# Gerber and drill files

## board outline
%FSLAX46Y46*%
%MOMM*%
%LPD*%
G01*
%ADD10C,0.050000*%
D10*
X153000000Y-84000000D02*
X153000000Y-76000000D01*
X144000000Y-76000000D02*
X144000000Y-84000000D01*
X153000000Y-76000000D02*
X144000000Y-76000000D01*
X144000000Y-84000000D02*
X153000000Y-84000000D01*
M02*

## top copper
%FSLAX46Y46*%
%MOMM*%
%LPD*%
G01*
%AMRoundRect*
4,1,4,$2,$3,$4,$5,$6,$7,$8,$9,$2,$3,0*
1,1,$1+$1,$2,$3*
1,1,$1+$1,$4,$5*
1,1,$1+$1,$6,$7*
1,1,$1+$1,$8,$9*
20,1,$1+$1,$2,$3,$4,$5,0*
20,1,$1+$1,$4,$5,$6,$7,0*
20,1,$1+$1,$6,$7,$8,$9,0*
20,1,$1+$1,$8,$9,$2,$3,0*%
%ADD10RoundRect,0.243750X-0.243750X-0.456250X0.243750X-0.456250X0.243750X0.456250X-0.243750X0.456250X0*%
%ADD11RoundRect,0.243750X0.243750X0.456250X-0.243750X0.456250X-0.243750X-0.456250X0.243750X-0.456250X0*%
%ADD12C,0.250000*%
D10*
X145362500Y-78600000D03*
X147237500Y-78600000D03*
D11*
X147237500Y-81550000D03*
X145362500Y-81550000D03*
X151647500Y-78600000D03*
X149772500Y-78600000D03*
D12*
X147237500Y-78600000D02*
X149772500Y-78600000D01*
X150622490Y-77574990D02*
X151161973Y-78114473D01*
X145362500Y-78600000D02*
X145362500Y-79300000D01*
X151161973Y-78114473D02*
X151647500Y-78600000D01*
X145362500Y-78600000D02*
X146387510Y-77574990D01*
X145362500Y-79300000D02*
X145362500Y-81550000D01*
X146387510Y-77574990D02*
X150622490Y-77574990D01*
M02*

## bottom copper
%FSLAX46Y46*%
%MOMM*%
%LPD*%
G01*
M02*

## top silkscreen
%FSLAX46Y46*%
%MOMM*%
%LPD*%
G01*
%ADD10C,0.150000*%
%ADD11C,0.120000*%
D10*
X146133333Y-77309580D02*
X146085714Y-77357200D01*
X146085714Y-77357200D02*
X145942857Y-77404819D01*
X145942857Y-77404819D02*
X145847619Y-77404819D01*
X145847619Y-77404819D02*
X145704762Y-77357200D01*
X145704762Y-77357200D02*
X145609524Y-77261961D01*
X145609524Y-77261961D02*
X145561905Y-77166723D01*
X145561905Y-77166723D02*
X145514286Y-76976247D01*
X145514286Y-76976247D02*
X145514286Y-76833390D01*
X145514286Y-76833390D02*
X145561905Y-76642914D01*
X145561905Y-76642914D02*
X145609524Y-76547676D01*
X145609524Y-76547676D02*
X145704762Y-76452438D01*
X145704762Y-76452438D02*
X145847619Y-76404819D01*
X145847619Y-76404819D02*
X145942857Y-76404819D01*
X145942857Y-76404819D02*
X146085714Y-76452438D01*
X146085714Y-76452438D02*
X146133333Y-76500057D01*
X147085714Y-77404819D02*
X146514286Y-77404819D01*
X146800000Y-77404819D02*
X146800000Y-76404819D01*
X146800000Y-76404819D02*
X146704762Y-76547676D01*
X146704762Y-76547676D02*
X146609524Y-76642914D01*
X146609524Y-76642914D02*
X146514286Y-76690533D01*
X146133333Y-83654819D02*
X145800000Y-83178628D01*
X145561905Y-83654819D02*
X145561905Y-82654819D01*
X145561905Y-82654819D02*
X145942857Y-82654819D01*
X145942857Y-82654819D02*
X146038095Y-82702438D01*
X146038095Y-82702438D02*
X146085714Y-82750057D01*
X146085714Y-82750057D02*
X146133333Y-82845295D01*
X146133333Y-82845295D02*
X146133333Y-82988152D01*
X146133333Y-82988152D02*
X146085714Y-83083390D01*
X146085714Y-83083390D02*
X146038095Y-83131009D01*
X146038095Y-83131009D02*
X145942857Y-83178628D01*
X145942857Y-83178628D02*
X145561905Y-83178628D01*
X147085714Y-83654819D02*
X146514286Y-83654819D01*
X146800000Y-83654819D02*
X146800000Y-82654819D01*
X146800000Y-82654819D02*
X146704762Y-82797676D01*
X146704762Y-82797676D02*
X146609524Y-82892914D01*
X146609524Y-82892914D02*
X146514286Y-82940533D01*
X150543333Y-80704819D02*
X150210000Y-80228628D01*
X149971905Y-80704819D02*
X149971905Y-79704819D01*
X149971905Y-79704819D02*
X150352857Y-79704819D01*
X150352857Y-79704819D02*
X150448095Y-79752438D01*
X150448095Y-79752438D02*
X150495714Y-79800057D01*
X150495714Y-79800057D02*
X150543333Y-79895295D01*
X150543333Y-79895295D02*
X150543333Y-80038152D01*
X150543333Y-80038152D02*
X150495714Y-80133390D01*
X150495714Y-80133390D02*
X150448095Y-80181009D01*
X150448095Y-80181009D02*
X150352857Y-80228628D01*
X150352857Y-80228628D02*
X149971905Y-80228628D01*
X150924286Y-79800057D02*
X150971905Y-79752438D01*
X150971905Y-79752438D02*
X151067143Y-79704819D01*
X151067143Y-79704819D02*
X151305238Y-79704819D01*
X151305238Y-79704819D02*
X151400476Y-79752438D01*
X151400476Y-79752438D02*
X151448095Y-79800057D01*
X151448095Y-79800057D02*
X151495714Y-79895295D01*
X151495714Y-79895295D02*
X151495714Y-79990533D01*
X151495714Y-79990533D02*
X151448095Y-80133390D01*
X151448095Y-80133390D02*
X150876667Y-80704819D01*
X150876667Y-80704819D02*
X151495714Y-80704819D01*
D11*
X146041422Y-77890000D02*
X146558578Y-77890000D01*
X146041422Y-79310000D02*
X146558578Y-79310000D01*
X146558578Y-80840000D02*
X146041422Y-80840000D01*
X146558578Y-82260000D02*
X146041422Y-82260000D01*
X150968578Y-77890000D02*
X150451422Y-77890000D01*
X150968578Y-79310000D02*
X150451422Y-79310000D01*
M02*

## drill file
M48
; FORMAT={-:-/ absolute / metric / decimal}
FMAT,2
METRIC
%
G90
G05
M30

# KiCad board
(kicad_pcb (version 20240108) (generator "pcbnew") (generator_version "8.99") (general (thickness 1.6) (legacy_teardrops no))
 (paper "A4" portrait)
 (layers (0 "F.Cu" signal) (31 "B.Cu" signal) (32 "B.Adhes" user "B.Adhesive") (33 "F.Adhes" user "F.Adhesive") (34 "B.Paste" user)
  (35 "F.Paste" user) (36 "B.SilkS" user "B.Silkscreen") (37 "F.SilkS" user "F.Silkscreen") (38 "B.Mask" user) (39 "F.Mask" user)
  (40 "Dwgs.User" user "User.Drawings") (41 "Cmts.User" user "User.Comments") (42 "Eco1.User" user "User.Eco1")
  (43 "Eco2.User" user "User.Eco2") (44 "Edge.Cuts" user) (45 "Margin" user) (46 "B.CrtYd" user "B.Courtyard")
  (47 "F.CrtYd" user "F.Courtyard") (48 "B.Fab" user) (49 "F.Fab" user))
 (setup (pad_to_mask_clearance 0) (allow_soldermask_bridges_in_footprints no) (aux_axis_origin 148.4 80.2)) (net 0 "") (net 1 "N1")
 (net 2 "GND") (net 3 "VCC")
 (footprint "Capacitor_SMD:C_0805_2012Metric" (layer "F.Cu") (at 146.3 78.6)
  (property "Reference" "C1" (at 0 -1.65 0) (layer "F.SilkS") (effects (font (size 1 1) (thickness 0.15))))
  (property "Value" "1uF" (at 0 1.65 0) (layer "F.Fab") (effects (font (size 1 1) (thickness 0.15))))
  (fp_line (start -0.258578 -0.71) (end 0.258578 -0.71) (stroke (width 0.12) (type solid)) (layer "F.SilkS"))
  (fp_line (start -0.258578 0.71) (end 0.258578 0.71) (stroke (width 0.12) (type solid)) (layer "F.SilkS"))
  (pad "1" smd roundrect (at -0.9375 0) (size 0.975 1.4) (layers "F.Cu" "F.Paste" "F.Mask") (roundrect_rratio 0.25) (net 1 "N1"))
  (pad "2" smd roundrect (at 0.9375 0) (size 0.975 1.4) (layers "F.Cu" "F.Paste" "F.Mask") (roundrect_rratio 0.25) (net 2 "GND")))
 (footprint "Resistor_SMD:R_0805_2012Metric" (layer "F.Cu") (at 146.3 81.55 180)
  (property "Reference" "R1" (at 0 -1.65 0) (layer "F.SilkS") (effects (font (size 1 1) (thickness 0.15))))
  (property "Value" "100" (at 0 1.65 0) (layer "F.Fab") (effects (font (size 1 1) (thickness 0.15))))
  (fp_line (start -0.258578 0.71) (end 0.258578 0.71) (stroke (width 0.12) (type solid)) (layer "F.SilkS"))
  (fp_line (start -0.258578 -0.71) (end 0.258578 -0.71) (stroke (width 0.12) (type solid)) (layer "F.SilkS"))
  (pad "1" smd roundrect (at -0.9375 0 180) (size 0.975 1.4) (layers "F.Cu" "F.Paste" "F.Mask") (roundrect_rratio 0.25) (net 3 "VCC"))
  (pad "2" smd roundrect (at 0.9375 0 180) (size 0.975 1.4) (layers "F.Cu" "F.Paste" "F.Mask") (roundrect_rratio 0.25) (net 1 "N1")))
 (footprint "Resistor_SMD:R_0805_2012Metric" (layer "F.Cu") (at 150.71 78.6 180)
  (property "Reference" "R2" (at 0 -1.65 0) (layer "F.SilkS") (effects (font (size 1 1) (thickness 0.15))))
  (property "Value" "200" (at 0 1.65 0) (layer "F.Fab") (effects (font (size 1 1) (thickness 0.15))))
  (fp_line (start -0.258578 0.71) (end 0.258578 0.71) (stroke (width 0.12) (type solid)) (layer "F.SilkS"))
  (fp_line (start -0.258578 -0.71) (end 0.258578 -0.71) (stroke (width 0.12) (type solid)) (layer "F.SilkS"))
  (pad "1" smd roundrect (at -0.9375 0 180) (size 0.975 1.4) (layers "F.Cu" "F.Paste" "F.Mask") (roundrect_rratio 0.25) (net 1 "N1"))
  (pad "2" smd roundrect (at 0.9375 0 180) (size 0.975 1.4) (layers "F.Cu" "F.Paste" "F.Mask") (roundrect_rratio 0.25) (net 2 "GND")))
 (gr_line (start 153 84) (end 153 76) (stroke (width 0.05) (type solid)) (layer "Edge.Cuts"))
 (gr_line (start 144 76) (end 144 84) (stroke (width 0.05) (type solid)) (layer "Edge.Cuts"))
 (gr_line (start 153 76) (end 144 76) (stroke (width 0.05) (type solid)) (layer "Edge.Cuts"))
 (gr_line (start 144 84) (end 153 84) (stroke (width 0.05) (type solid)) (layer "Edge.Cuts"))
 (segment (start 147.2375 78.6) (end 149.7725 78.6) (width 0.25) (layer "F.Cu") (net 2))
 (segment (start 150.62249 77.57499) (end 151.161973 78.114473) (width 0.25) (layer "F.Cu") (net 1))
 (segment (start 145.3625 78.6) (end 145.3625 79.3) (width 0.25) (layer "F.Cu") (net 1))
 (segment (start 151.161973 78.114473) (end 151.6475 78.6) (width 0.25) (layer "F.Cu") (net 1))
 (segment (start 145.3625 78.6) (end 146.38751 77.57499) (width 0.25) (layer "F.Cu") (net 1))
 (segment (start 145.3625 79.3) (end 145.3625 81.55) (width 0.25) (layer "F.Cu") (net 1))
 (segment (start 146.38751 77.57499) (end 150.62249 77.57499) (width 0.25) (layer "F.Cu") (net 1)))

